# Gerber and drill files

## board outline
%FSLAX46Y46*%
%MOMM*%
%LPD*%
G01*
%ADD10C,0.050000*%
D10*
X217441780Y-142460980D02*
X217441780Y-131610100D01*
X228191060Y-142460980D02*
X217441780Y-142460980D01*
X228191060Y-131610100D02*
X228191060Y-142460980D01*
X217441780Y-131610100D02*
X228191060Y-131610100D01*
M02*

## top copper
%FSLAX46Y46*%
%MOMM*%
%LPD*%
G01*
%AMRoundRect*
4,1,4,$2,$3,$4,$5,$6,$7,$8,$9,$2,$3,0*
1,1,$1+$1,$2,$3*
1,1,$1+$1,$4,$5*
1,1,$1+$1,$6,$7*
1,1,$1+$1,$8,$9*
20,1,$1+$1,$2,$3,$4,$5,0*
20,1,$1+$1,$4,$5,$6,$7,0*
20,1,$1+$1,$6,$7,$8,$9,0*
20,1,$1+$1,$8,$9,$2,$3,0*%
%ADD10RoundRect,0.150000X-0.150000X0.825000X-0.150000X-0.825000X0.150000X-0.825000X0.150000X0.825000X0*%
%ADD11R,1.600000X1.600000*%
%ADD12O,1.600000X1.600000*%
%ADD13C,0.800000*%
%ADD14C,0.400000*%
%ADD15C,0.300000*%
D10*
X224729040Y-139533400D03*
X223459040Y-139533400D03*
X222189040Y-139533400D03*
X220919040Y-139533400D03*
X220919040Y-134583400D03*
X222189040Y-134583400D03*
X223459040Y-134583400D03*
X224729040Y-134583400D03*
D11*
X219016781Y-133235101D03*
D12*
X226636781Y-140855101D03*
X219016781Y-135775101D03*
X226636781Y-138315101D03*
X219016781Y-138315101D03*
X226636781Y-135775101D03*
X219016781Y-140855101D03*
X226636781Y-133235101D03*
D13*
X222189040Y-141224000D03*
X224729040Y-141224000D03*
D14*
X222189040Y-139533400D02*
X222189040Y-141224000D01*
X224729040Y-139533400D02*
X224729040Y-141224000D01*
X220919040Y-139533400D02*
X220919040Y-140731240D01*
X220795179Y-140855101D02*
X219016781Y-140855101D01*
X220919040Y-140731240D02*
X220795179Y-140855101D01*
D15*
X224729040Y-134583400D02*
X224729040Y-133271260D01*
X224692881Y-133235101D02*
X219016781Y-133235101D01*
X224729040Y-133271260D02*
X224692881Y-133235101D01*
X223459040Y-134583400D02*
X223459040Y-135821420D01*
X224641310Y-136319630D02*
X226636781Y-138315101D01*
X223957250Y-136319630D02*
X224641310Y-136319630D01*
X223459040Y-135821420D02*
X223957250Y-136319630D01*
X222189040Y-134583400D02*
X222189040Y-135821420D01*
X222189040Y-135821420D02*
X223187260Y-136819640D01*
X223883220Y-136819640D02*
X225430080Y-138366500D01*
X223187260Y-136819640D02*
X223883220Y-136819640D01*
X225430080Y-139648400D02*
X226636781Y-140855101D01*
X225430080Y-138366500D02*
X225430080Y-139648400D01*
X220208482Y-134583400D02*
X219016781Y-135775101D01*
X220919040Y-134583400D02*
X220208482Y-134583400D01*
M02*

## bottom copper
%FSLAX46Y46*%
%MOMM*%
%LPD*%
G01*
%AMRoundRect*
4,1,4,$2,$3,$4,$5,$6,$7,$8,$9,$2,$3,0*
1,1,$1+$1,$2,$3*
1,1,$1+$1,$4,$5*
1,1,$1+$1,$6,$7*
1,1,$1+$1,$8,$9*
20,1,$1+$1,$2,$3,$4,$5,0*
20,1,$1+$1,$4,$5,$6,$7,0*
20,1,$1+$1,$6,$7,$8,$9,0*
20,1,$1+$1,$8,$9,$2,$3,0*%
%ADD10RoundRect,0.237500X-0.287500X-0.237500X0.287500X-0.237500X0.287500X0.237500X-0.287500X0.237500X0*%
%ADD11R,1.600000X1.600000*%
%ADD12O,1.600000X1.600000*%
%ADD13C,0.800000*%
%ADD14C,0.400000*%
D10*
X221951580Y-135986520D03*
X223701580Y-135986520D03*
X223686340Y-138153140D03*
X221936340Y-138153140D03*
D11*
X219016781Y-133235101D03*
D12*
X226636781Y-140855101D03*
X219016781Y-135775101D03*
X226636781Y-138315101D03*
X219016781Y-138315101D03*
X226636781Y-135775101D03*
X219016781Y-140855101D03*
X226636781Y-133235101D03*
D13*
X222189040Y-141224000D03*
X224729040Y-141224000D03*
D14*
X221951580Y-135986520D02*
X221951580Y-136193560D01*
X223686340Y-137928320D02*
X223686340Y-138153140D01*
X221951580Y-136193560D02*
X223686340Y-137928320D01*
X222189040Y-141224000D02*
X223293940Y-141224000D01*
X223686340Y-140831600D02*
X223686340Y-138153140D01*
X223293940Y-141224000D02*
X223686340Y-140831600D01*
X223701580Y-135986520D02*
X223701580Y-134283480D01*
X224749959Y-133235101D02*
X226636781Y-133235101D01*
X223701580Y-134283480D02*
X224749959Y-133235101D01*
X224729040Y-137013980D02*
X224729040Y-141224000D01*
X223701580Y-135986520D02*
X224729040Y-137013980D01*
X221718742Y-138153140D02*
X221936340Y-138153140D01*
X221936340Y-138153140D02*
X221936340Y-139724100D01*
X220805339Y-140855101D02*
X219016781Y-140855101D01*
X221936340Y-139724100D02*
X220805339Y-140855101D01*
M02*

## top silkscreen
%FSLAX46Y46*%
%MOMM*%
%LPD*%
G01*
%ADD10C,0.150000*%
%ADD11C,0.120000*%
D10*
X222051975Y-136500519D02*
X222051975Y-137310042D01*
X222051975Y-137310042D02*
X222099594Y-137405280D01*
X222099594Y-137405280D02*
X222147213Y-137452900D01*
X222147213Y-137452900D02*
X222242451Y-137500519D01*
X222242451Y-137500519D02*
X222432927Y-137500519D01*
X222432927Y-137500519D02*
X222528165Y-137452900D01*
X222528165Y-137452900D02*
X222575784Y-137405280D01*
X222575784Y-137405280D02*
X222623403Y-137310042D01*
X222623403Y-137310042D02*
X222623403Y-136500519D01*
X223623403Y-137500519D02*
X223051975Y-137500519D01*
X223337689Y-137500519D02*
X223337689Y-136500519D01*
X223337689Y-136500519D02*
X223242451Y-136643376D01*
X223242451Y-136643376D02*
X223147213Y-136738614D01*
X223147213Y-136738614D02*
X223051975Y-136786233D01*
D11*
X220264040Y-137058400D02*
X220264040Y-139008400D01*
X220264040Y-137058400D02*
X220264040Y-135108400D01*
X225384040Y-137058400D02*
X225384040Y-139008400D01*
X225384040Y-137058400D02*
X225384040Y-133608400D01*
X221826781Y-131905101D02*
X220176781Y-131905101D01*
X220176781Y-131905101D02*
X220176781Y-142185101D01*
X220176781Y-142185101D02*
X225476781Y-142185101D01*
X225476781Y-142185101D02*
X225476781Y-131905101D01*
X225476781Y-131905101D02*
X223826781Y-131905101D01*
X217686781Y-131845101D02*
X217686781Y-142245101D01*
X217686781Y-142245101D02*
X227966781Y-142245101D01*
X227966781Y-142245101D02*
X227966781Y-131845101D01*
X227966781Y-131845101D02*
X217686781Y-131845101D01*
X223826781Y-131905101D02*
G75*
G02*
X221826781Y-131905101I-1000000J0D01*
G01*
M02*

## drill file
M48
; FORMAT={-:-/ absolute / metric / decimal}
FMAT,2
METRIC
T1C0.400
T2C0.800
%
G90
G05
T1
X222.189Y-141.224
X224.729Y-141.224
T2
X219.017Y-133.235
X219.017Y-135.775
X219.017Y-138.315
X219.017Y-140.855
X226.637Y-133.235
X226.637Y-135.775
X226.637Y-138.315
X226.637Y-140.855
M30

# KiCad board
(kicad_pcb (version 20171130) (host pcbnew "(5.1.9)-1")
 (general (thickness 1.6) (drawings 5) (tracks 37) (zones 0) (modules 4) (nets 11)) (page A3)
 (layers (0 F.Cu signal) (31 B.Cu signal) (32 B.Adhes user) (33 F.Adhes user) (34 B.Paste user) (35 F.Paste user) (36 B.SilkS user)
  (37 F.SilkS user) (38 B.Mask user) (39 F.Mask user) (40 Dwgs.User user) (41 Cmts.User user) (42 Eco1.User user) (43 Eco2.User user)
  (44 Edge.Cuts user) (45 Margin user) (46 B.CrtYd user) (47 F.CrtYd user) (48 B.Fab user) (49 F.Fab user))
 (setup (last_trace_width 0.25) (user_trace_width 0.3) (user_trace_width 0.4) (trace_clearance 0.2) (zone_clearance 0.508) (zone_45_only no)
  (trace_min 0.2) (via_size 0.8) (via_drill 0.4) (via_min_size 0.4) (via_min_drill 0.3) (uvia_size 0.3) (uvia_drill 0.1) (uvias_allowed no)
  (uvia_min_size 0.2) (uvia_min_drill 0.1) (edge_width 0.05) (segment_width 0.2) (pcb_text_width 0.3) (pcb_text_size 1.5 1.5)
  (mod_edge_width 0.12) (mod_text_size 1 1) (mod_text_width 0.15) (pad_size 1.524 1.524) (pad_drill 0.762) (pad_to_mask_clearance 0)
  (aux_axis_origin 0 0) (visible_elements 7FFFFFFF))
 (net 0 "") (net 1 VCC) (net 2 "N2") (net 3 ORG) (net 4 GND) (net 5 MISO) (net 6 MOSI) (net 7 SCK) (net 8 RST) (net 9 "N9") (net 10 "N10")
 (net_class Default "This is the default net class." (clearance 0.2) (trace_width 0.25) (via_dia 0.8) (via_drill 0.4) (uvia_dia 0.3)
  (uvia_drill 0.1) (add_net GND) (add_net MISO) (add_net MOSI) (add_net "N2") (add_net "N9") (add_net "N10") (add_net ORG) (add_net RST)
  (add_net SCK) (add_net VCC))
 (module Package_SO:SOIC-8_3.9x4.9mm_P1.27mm (layer F.Cu) (at 222.82404 137.0584 270)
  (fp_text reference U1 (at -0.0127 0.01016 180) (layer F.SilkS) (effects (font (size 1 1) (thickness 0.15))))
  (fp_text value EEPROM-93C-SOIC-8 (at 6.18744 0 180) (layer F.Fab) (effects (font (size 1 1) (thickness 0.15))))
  (fp_line (start 0 2.56) (end 1.95 2.56) (layer F.SilkS) (width 0.12))
  (fp_line (start 0 2.56) (end -1.95 2.56) (layer F.SilkS) (width 0.12))
  (fp_line (start 0 -2.56) (end 1.95 -2.56) (layer F.SilkS) (width 0.12))
  (fp_line (start 0 -2.56) (end -3.45 -2.56) (layer F.SilkS) (width 0.12))
  (pad 8 smd roundrect (at 2.475 -1.905 270) (size 1.95 0.6) (layers F.Cu F.Paste F.Mask) (roundrect_rratio 0.25) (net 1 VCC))
  (pad 7 smd roundrect (at 2.475 -0.635 270) (size 1.95 0.6) (layers F.Cu F.Paste F.Mask) (roundrect_rratio 0.25) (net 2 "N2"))
  (pad 6 smd roundrect (at 2.475 0.635 270) (size 1.95 0.6) (layers F.Cu F.Paste F.Mask) (roundrect_rratio 0.25) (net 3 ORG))
  (pad 5 smd roundrect (at 2.475 1.905 270) (size 1.95 0.6) (layers F.Cu F.Paste F.Mask) (roundrect_rratio 0.25) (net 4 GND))
  (pad 4 smd roundrect (at -2.475 1.905 270) (size 1.95 0.6) (layers F.Cu F.Paste F.Mask) (roundrect_rratio 0.25) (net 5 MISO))
  (pad 3 smd roundrect (at -2.475 0.635 270) (size 1.95 0.6) (layers F.Cu F.Paste F.Mask) (roundrect_rratio 0.25) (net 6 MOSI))
  (pad 2 smd roundrect (at -2.475 -0.635 270) (size 1.95 0.6) (layers F.Cu F.Paste F.Mask) (roundrect_rratio 0.25) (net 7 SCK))
  (pad 1 smd roundrect (at -2.475 -1.905 270) (size 1.95 0.6) (layers F.Cu F.Paste F.Mask) (roundrect_rratio 0.25) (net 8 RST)))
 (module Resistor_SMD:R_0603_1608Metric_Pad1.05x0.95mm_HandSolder (layer B.Cu) (at 222.82658 135.98652)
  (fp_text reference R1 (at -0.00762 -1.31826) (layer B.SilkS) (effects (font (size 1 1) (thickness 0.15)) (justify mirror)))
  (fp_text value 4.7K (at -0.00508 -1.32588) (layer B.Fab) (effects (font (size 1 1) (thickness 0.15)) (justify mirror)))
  (pad 1 smd roundrect (at -0.875 0) (size 1.05 0.95) (layers B.Cu B.Paste B.Mask) (roundrect_rratio 0.25) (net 3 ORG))
  (pad 2 smd roundrect (at 0.875 0) (size 1.05 0.95) (layers B.Cu B.Paste B.Mask) (roundrect_rratio 0.25) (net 1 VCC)))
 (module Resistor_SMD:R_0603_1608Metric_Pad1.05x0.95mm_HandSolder (layer B.Cu) (at 222.81134 138.15314)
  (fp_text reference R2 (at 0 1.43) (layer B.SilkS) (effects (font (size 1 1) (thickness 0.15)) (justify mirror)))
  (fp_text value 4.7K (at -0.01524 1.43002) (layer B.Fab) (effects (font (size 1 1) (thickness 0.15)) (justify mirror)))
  (pad 2 smd roundrect (at 0.875 0) (size 1.05 0.95) (layers B.Cu B.Paste B.Mask) (roundrect_rratio 0.25) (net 3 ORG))
  (pad 1 smd roundrect (at -0.875 0) (size 1.05 0.95) (layers B.Cu B.Paste B.Mask) (roundrect_rratio 0.25) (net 4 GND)))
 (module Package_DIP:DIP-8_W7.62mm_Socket (layer F.Cu) (at 219.016781 133.235101)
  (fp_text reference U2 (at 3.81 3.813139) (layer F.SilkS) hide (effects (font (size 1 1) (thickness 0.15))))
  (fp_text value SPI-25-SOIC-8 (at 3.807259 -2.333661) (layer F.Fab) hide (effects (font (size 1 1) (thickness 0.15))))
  (fp_line (start 2.81 -1.33) (end 1.16 -1.33) (layer F.SilkS) (width 0.12))
  (fp_line (start 1.16 -1.33) (end 1.16 8.95) (layer F.SilkS) (width 0.12))
  (fp_line (start 1.16 8.95) (end 6.46 8.95) (layer F.SilkS) (width 0.12))
  (fp_line (start 6.46 8.95) (end 6.46 -1.33) (layer F.SilkS) (width 0.12))
  (fp_line (start 6.46 -1.33) (end 4.81 -1.33) (layer F.SilkS) (width 0.12))
  (fp_line (start -1.33 -1.39) (end -1.33 9.01) (layer F.SilkS) (width 0.12))
  (fp_line (start -1.33 9.01) (end 8.95 9.01) (layer F.SilkS) (width 0.12))
  (fp_line (start 8.95 9.01) (end 8.95 -1.39) (layer F.SilkS) (width 0.12))
  (fp_line (start 8.95 -1.39) (end -1.33 -1.39) (layer F.SilkS) (width 0.12))
  (fp_arc (start 3.81 -1.33) (end 2.81 -1.33) (angle -180) (layer F.SilkS) (width 0.12))
  (pad 1 thru_hole rect (at 0 0) (size 1.6 1.6) (drill 0.8) (layers *.Cu *.Mask) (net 8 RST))
  (pad 5 thru_hole oval (at 7.62 7.62) (size 1.6 1.6) (drill 0.8) (layers *.Cu *.Mask) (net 6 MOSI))
  (pad 2 thru_hole oval (at 0 2.54) (size 1.6 1.6) (drill 0.8) (layers *.Cu *.Mask) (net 5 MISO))
  (pad 6 thru_hole oval (at 7.62 5.08) (size 1.6 1.6) (drill 0.8) (layers *.Cu *.Mask) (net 7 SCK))
  (pad 3 thru_hole oval (at 0 5.08) (size 1.6 1.6) (drill 0.8) (layers *.Cu *.Mask) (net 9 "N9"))
  (pad 7 thru_hole oval (at 7.62 2.54) (size 1.6 1.6) (drill 0.8) (layers *.Cu *.Mask) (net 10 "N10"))
  (pad 4 thru_hole oval (at 0 7.62) (size 1.6 1.6) (drill 0.8) (layers *.Cu *.Mask) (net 4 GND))
  (pad 8 thru_hole oval (at 7.62 0) (size 1.6 1.6) (drill 0.8) (layers *.Cu *.Mask) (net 1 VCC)))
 (gr_line (start 217.44178 142.46098) (end 217.44178 131.6101) (layer Edge.Cuts) (width 0.05))
 (gr_line (start 228.19106 142.46098) (end 217.44178 142.46098) (layer Edge.Cuts) (width 0.05))
 (gr_line (start 228.19106 131.6101) (end 228.19106 142.46098) (layer Edge.Cuts) (width 0.05))
 (gr_line (start 217.44178 131.6101) (end 228.19106 131.6101) (layer Edge.Cuts) (width 0.05))
 (segment (start 221.95158 135.98652) (end 221.95158 136.19356) (width 0.4) (layer B.Cu) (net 3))
 (segment (start 223.68634 137.92832) (end 223.68634 138.15314) (width 0.4) (layer B.Cu) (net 3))
 (segment (start 221.95158 136.19356) (end 223.68634 137.92832) (width 0.4) (layer B.Cu) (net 3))
 (segment (start 222.18904 139.5334) (end 222.18904 141.224) (width 0.4) (layer F.Cu) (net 3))
 (via (at 222.18904 141.224) (size 0.8) (drill 0.4) (layers F.Cu B.Cu) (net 3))
 (segment (start 222.18904 141.224) (end 223.29394 141.224) (width 0.4) (layer B.Cu) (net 3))
 (segment (start 223.68634 140.8316) (end 223.68634 138.15314) (width 0.4) (layer B.Cu) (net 3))
 (segment (start 223.29394 141.224) (end 223.68634 140.8316) (width 0.4) (layer B.Cu) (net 3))
 (segment (start 223.70158 135.98652) (end 223.70158 134.28348) (width 0.4) (layer B.Cu) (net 1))
 (segment (start 224.749959 133.235101) (end 226.636781 133.235101) (width 0.4) (layer B.Cu) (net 1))
 (segment (start 223.70158 134.28348) (end 224.749959 133.235101) (width 0.4) (layer B.Cu) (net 1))
 (segment (start 224.72904 139.5334) (end 224.72904 141.224) (width 0.4) (layer F.Cu) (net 1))
 (via (at 224.72904 141.224) (size 0.8) (drill 0.4) (layers F.Cu B.Cu) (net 1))
 (segment (start 224.72904 137.01398) (end 224.72904 141.224) (width 0.4) (layer B.Cu) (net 1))
 (segment (start 223.70158 135.98652) (end 224.72904 137.01398) (width 0.4) (layer B.Cu) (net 1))
 (segment (start 221.718742 138.15314) (end 221.93634 138.15314) (width 0.4) (layer B.Cu) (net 4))
 (segment (start 220.91904 139.5334) (end 220.91904 140.73124) (width 0.4) (layer F.Cu) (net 4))
 (segment (start 220.795179 140.855101) (end 219.016781 140.855101) (width 0.4) (layer F.Cu) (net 4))
 (segment (start 220.91904 140.73124) (end 220.795179 140.855101) (width 0.4) (layer F.Cu) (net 4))
 (segment (start 221.93634 138.15314) (end 221.93634 139.7241) (width 0.4) (layer B.Cu) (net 4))
 (segment (start 220.805339 140.855101) (end 219.016781 140.855101) (width 0.4) (layer B.Cu) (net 4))
 (segment (start 221.93634 139.7241) (end 220.805339 140.855101) (width 0.4) (layer B.Cu) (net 4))
 (segment (start 224.72904 134.5834) (end 224.72904 133.27126) (width 0.3) (layer F.Cu) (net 8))
 (segment (start 224.692881 133.235101) (end 219.016781 133.235101) (width 0.3) (layer F.Cu) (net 8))
 (segment (start 224.72904 133.27126) (end 224.692881 133.235101) (width 0.3) (layer F.Cu) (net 8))
 (segment (start 223.45904 134.5834) (end 223.45904 135.82142) (width 0.3) (layer F.Cu) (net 7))
 (segment (start 224.64131 136.31963) (end 226.636781 138.315101) (width 0.3) (layer F.Cu) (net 7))
 (segment (start 223.95725 136.31963) (end 224.64131 136.31963) (width 0.3) (layer F.Cu) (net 7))
 (segment (start 223.45904 135.82142) (end 223.95725 136.31963) (width 0.3) (layer F.Cu) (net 7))
 (segment (start 222.18904 134.5834) (end 222.18904 135.82142) (width 0.3) (layer F.Cu) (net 6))
 (segment (start 222.18904 135.82142) (end 223.18726 136.81964) (width 0.3) (layer F.Cu) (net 6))
 (segment (start 223.88322 136.81964) (end 225.43008 138.3665) (width 0.3) (layer F.Cu) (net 6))
 (segment (start 223.18726 136.81964) (end 223.88322 136.81964) (width 0.3) (layer F.Cu) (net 6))
 (segment (start 225.43008 139.6484) (end 226.636781 140.855101) (width 0.3) (layer F.Cu) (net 6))
 (segment (start 225.43008 138.3665) (end 225.43008 139.6484) (width 0.3) (layer F.Cu) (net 6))
 (segment (start 220.208482 134.5834) (end 219.016781 135.775101) (width 0.3) (layer F.Cu) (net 5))
 (segment (start 220.91904 134.5834) (end 220.208482 134.5834) (width 0.3) (layer F.Cu) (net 5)))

